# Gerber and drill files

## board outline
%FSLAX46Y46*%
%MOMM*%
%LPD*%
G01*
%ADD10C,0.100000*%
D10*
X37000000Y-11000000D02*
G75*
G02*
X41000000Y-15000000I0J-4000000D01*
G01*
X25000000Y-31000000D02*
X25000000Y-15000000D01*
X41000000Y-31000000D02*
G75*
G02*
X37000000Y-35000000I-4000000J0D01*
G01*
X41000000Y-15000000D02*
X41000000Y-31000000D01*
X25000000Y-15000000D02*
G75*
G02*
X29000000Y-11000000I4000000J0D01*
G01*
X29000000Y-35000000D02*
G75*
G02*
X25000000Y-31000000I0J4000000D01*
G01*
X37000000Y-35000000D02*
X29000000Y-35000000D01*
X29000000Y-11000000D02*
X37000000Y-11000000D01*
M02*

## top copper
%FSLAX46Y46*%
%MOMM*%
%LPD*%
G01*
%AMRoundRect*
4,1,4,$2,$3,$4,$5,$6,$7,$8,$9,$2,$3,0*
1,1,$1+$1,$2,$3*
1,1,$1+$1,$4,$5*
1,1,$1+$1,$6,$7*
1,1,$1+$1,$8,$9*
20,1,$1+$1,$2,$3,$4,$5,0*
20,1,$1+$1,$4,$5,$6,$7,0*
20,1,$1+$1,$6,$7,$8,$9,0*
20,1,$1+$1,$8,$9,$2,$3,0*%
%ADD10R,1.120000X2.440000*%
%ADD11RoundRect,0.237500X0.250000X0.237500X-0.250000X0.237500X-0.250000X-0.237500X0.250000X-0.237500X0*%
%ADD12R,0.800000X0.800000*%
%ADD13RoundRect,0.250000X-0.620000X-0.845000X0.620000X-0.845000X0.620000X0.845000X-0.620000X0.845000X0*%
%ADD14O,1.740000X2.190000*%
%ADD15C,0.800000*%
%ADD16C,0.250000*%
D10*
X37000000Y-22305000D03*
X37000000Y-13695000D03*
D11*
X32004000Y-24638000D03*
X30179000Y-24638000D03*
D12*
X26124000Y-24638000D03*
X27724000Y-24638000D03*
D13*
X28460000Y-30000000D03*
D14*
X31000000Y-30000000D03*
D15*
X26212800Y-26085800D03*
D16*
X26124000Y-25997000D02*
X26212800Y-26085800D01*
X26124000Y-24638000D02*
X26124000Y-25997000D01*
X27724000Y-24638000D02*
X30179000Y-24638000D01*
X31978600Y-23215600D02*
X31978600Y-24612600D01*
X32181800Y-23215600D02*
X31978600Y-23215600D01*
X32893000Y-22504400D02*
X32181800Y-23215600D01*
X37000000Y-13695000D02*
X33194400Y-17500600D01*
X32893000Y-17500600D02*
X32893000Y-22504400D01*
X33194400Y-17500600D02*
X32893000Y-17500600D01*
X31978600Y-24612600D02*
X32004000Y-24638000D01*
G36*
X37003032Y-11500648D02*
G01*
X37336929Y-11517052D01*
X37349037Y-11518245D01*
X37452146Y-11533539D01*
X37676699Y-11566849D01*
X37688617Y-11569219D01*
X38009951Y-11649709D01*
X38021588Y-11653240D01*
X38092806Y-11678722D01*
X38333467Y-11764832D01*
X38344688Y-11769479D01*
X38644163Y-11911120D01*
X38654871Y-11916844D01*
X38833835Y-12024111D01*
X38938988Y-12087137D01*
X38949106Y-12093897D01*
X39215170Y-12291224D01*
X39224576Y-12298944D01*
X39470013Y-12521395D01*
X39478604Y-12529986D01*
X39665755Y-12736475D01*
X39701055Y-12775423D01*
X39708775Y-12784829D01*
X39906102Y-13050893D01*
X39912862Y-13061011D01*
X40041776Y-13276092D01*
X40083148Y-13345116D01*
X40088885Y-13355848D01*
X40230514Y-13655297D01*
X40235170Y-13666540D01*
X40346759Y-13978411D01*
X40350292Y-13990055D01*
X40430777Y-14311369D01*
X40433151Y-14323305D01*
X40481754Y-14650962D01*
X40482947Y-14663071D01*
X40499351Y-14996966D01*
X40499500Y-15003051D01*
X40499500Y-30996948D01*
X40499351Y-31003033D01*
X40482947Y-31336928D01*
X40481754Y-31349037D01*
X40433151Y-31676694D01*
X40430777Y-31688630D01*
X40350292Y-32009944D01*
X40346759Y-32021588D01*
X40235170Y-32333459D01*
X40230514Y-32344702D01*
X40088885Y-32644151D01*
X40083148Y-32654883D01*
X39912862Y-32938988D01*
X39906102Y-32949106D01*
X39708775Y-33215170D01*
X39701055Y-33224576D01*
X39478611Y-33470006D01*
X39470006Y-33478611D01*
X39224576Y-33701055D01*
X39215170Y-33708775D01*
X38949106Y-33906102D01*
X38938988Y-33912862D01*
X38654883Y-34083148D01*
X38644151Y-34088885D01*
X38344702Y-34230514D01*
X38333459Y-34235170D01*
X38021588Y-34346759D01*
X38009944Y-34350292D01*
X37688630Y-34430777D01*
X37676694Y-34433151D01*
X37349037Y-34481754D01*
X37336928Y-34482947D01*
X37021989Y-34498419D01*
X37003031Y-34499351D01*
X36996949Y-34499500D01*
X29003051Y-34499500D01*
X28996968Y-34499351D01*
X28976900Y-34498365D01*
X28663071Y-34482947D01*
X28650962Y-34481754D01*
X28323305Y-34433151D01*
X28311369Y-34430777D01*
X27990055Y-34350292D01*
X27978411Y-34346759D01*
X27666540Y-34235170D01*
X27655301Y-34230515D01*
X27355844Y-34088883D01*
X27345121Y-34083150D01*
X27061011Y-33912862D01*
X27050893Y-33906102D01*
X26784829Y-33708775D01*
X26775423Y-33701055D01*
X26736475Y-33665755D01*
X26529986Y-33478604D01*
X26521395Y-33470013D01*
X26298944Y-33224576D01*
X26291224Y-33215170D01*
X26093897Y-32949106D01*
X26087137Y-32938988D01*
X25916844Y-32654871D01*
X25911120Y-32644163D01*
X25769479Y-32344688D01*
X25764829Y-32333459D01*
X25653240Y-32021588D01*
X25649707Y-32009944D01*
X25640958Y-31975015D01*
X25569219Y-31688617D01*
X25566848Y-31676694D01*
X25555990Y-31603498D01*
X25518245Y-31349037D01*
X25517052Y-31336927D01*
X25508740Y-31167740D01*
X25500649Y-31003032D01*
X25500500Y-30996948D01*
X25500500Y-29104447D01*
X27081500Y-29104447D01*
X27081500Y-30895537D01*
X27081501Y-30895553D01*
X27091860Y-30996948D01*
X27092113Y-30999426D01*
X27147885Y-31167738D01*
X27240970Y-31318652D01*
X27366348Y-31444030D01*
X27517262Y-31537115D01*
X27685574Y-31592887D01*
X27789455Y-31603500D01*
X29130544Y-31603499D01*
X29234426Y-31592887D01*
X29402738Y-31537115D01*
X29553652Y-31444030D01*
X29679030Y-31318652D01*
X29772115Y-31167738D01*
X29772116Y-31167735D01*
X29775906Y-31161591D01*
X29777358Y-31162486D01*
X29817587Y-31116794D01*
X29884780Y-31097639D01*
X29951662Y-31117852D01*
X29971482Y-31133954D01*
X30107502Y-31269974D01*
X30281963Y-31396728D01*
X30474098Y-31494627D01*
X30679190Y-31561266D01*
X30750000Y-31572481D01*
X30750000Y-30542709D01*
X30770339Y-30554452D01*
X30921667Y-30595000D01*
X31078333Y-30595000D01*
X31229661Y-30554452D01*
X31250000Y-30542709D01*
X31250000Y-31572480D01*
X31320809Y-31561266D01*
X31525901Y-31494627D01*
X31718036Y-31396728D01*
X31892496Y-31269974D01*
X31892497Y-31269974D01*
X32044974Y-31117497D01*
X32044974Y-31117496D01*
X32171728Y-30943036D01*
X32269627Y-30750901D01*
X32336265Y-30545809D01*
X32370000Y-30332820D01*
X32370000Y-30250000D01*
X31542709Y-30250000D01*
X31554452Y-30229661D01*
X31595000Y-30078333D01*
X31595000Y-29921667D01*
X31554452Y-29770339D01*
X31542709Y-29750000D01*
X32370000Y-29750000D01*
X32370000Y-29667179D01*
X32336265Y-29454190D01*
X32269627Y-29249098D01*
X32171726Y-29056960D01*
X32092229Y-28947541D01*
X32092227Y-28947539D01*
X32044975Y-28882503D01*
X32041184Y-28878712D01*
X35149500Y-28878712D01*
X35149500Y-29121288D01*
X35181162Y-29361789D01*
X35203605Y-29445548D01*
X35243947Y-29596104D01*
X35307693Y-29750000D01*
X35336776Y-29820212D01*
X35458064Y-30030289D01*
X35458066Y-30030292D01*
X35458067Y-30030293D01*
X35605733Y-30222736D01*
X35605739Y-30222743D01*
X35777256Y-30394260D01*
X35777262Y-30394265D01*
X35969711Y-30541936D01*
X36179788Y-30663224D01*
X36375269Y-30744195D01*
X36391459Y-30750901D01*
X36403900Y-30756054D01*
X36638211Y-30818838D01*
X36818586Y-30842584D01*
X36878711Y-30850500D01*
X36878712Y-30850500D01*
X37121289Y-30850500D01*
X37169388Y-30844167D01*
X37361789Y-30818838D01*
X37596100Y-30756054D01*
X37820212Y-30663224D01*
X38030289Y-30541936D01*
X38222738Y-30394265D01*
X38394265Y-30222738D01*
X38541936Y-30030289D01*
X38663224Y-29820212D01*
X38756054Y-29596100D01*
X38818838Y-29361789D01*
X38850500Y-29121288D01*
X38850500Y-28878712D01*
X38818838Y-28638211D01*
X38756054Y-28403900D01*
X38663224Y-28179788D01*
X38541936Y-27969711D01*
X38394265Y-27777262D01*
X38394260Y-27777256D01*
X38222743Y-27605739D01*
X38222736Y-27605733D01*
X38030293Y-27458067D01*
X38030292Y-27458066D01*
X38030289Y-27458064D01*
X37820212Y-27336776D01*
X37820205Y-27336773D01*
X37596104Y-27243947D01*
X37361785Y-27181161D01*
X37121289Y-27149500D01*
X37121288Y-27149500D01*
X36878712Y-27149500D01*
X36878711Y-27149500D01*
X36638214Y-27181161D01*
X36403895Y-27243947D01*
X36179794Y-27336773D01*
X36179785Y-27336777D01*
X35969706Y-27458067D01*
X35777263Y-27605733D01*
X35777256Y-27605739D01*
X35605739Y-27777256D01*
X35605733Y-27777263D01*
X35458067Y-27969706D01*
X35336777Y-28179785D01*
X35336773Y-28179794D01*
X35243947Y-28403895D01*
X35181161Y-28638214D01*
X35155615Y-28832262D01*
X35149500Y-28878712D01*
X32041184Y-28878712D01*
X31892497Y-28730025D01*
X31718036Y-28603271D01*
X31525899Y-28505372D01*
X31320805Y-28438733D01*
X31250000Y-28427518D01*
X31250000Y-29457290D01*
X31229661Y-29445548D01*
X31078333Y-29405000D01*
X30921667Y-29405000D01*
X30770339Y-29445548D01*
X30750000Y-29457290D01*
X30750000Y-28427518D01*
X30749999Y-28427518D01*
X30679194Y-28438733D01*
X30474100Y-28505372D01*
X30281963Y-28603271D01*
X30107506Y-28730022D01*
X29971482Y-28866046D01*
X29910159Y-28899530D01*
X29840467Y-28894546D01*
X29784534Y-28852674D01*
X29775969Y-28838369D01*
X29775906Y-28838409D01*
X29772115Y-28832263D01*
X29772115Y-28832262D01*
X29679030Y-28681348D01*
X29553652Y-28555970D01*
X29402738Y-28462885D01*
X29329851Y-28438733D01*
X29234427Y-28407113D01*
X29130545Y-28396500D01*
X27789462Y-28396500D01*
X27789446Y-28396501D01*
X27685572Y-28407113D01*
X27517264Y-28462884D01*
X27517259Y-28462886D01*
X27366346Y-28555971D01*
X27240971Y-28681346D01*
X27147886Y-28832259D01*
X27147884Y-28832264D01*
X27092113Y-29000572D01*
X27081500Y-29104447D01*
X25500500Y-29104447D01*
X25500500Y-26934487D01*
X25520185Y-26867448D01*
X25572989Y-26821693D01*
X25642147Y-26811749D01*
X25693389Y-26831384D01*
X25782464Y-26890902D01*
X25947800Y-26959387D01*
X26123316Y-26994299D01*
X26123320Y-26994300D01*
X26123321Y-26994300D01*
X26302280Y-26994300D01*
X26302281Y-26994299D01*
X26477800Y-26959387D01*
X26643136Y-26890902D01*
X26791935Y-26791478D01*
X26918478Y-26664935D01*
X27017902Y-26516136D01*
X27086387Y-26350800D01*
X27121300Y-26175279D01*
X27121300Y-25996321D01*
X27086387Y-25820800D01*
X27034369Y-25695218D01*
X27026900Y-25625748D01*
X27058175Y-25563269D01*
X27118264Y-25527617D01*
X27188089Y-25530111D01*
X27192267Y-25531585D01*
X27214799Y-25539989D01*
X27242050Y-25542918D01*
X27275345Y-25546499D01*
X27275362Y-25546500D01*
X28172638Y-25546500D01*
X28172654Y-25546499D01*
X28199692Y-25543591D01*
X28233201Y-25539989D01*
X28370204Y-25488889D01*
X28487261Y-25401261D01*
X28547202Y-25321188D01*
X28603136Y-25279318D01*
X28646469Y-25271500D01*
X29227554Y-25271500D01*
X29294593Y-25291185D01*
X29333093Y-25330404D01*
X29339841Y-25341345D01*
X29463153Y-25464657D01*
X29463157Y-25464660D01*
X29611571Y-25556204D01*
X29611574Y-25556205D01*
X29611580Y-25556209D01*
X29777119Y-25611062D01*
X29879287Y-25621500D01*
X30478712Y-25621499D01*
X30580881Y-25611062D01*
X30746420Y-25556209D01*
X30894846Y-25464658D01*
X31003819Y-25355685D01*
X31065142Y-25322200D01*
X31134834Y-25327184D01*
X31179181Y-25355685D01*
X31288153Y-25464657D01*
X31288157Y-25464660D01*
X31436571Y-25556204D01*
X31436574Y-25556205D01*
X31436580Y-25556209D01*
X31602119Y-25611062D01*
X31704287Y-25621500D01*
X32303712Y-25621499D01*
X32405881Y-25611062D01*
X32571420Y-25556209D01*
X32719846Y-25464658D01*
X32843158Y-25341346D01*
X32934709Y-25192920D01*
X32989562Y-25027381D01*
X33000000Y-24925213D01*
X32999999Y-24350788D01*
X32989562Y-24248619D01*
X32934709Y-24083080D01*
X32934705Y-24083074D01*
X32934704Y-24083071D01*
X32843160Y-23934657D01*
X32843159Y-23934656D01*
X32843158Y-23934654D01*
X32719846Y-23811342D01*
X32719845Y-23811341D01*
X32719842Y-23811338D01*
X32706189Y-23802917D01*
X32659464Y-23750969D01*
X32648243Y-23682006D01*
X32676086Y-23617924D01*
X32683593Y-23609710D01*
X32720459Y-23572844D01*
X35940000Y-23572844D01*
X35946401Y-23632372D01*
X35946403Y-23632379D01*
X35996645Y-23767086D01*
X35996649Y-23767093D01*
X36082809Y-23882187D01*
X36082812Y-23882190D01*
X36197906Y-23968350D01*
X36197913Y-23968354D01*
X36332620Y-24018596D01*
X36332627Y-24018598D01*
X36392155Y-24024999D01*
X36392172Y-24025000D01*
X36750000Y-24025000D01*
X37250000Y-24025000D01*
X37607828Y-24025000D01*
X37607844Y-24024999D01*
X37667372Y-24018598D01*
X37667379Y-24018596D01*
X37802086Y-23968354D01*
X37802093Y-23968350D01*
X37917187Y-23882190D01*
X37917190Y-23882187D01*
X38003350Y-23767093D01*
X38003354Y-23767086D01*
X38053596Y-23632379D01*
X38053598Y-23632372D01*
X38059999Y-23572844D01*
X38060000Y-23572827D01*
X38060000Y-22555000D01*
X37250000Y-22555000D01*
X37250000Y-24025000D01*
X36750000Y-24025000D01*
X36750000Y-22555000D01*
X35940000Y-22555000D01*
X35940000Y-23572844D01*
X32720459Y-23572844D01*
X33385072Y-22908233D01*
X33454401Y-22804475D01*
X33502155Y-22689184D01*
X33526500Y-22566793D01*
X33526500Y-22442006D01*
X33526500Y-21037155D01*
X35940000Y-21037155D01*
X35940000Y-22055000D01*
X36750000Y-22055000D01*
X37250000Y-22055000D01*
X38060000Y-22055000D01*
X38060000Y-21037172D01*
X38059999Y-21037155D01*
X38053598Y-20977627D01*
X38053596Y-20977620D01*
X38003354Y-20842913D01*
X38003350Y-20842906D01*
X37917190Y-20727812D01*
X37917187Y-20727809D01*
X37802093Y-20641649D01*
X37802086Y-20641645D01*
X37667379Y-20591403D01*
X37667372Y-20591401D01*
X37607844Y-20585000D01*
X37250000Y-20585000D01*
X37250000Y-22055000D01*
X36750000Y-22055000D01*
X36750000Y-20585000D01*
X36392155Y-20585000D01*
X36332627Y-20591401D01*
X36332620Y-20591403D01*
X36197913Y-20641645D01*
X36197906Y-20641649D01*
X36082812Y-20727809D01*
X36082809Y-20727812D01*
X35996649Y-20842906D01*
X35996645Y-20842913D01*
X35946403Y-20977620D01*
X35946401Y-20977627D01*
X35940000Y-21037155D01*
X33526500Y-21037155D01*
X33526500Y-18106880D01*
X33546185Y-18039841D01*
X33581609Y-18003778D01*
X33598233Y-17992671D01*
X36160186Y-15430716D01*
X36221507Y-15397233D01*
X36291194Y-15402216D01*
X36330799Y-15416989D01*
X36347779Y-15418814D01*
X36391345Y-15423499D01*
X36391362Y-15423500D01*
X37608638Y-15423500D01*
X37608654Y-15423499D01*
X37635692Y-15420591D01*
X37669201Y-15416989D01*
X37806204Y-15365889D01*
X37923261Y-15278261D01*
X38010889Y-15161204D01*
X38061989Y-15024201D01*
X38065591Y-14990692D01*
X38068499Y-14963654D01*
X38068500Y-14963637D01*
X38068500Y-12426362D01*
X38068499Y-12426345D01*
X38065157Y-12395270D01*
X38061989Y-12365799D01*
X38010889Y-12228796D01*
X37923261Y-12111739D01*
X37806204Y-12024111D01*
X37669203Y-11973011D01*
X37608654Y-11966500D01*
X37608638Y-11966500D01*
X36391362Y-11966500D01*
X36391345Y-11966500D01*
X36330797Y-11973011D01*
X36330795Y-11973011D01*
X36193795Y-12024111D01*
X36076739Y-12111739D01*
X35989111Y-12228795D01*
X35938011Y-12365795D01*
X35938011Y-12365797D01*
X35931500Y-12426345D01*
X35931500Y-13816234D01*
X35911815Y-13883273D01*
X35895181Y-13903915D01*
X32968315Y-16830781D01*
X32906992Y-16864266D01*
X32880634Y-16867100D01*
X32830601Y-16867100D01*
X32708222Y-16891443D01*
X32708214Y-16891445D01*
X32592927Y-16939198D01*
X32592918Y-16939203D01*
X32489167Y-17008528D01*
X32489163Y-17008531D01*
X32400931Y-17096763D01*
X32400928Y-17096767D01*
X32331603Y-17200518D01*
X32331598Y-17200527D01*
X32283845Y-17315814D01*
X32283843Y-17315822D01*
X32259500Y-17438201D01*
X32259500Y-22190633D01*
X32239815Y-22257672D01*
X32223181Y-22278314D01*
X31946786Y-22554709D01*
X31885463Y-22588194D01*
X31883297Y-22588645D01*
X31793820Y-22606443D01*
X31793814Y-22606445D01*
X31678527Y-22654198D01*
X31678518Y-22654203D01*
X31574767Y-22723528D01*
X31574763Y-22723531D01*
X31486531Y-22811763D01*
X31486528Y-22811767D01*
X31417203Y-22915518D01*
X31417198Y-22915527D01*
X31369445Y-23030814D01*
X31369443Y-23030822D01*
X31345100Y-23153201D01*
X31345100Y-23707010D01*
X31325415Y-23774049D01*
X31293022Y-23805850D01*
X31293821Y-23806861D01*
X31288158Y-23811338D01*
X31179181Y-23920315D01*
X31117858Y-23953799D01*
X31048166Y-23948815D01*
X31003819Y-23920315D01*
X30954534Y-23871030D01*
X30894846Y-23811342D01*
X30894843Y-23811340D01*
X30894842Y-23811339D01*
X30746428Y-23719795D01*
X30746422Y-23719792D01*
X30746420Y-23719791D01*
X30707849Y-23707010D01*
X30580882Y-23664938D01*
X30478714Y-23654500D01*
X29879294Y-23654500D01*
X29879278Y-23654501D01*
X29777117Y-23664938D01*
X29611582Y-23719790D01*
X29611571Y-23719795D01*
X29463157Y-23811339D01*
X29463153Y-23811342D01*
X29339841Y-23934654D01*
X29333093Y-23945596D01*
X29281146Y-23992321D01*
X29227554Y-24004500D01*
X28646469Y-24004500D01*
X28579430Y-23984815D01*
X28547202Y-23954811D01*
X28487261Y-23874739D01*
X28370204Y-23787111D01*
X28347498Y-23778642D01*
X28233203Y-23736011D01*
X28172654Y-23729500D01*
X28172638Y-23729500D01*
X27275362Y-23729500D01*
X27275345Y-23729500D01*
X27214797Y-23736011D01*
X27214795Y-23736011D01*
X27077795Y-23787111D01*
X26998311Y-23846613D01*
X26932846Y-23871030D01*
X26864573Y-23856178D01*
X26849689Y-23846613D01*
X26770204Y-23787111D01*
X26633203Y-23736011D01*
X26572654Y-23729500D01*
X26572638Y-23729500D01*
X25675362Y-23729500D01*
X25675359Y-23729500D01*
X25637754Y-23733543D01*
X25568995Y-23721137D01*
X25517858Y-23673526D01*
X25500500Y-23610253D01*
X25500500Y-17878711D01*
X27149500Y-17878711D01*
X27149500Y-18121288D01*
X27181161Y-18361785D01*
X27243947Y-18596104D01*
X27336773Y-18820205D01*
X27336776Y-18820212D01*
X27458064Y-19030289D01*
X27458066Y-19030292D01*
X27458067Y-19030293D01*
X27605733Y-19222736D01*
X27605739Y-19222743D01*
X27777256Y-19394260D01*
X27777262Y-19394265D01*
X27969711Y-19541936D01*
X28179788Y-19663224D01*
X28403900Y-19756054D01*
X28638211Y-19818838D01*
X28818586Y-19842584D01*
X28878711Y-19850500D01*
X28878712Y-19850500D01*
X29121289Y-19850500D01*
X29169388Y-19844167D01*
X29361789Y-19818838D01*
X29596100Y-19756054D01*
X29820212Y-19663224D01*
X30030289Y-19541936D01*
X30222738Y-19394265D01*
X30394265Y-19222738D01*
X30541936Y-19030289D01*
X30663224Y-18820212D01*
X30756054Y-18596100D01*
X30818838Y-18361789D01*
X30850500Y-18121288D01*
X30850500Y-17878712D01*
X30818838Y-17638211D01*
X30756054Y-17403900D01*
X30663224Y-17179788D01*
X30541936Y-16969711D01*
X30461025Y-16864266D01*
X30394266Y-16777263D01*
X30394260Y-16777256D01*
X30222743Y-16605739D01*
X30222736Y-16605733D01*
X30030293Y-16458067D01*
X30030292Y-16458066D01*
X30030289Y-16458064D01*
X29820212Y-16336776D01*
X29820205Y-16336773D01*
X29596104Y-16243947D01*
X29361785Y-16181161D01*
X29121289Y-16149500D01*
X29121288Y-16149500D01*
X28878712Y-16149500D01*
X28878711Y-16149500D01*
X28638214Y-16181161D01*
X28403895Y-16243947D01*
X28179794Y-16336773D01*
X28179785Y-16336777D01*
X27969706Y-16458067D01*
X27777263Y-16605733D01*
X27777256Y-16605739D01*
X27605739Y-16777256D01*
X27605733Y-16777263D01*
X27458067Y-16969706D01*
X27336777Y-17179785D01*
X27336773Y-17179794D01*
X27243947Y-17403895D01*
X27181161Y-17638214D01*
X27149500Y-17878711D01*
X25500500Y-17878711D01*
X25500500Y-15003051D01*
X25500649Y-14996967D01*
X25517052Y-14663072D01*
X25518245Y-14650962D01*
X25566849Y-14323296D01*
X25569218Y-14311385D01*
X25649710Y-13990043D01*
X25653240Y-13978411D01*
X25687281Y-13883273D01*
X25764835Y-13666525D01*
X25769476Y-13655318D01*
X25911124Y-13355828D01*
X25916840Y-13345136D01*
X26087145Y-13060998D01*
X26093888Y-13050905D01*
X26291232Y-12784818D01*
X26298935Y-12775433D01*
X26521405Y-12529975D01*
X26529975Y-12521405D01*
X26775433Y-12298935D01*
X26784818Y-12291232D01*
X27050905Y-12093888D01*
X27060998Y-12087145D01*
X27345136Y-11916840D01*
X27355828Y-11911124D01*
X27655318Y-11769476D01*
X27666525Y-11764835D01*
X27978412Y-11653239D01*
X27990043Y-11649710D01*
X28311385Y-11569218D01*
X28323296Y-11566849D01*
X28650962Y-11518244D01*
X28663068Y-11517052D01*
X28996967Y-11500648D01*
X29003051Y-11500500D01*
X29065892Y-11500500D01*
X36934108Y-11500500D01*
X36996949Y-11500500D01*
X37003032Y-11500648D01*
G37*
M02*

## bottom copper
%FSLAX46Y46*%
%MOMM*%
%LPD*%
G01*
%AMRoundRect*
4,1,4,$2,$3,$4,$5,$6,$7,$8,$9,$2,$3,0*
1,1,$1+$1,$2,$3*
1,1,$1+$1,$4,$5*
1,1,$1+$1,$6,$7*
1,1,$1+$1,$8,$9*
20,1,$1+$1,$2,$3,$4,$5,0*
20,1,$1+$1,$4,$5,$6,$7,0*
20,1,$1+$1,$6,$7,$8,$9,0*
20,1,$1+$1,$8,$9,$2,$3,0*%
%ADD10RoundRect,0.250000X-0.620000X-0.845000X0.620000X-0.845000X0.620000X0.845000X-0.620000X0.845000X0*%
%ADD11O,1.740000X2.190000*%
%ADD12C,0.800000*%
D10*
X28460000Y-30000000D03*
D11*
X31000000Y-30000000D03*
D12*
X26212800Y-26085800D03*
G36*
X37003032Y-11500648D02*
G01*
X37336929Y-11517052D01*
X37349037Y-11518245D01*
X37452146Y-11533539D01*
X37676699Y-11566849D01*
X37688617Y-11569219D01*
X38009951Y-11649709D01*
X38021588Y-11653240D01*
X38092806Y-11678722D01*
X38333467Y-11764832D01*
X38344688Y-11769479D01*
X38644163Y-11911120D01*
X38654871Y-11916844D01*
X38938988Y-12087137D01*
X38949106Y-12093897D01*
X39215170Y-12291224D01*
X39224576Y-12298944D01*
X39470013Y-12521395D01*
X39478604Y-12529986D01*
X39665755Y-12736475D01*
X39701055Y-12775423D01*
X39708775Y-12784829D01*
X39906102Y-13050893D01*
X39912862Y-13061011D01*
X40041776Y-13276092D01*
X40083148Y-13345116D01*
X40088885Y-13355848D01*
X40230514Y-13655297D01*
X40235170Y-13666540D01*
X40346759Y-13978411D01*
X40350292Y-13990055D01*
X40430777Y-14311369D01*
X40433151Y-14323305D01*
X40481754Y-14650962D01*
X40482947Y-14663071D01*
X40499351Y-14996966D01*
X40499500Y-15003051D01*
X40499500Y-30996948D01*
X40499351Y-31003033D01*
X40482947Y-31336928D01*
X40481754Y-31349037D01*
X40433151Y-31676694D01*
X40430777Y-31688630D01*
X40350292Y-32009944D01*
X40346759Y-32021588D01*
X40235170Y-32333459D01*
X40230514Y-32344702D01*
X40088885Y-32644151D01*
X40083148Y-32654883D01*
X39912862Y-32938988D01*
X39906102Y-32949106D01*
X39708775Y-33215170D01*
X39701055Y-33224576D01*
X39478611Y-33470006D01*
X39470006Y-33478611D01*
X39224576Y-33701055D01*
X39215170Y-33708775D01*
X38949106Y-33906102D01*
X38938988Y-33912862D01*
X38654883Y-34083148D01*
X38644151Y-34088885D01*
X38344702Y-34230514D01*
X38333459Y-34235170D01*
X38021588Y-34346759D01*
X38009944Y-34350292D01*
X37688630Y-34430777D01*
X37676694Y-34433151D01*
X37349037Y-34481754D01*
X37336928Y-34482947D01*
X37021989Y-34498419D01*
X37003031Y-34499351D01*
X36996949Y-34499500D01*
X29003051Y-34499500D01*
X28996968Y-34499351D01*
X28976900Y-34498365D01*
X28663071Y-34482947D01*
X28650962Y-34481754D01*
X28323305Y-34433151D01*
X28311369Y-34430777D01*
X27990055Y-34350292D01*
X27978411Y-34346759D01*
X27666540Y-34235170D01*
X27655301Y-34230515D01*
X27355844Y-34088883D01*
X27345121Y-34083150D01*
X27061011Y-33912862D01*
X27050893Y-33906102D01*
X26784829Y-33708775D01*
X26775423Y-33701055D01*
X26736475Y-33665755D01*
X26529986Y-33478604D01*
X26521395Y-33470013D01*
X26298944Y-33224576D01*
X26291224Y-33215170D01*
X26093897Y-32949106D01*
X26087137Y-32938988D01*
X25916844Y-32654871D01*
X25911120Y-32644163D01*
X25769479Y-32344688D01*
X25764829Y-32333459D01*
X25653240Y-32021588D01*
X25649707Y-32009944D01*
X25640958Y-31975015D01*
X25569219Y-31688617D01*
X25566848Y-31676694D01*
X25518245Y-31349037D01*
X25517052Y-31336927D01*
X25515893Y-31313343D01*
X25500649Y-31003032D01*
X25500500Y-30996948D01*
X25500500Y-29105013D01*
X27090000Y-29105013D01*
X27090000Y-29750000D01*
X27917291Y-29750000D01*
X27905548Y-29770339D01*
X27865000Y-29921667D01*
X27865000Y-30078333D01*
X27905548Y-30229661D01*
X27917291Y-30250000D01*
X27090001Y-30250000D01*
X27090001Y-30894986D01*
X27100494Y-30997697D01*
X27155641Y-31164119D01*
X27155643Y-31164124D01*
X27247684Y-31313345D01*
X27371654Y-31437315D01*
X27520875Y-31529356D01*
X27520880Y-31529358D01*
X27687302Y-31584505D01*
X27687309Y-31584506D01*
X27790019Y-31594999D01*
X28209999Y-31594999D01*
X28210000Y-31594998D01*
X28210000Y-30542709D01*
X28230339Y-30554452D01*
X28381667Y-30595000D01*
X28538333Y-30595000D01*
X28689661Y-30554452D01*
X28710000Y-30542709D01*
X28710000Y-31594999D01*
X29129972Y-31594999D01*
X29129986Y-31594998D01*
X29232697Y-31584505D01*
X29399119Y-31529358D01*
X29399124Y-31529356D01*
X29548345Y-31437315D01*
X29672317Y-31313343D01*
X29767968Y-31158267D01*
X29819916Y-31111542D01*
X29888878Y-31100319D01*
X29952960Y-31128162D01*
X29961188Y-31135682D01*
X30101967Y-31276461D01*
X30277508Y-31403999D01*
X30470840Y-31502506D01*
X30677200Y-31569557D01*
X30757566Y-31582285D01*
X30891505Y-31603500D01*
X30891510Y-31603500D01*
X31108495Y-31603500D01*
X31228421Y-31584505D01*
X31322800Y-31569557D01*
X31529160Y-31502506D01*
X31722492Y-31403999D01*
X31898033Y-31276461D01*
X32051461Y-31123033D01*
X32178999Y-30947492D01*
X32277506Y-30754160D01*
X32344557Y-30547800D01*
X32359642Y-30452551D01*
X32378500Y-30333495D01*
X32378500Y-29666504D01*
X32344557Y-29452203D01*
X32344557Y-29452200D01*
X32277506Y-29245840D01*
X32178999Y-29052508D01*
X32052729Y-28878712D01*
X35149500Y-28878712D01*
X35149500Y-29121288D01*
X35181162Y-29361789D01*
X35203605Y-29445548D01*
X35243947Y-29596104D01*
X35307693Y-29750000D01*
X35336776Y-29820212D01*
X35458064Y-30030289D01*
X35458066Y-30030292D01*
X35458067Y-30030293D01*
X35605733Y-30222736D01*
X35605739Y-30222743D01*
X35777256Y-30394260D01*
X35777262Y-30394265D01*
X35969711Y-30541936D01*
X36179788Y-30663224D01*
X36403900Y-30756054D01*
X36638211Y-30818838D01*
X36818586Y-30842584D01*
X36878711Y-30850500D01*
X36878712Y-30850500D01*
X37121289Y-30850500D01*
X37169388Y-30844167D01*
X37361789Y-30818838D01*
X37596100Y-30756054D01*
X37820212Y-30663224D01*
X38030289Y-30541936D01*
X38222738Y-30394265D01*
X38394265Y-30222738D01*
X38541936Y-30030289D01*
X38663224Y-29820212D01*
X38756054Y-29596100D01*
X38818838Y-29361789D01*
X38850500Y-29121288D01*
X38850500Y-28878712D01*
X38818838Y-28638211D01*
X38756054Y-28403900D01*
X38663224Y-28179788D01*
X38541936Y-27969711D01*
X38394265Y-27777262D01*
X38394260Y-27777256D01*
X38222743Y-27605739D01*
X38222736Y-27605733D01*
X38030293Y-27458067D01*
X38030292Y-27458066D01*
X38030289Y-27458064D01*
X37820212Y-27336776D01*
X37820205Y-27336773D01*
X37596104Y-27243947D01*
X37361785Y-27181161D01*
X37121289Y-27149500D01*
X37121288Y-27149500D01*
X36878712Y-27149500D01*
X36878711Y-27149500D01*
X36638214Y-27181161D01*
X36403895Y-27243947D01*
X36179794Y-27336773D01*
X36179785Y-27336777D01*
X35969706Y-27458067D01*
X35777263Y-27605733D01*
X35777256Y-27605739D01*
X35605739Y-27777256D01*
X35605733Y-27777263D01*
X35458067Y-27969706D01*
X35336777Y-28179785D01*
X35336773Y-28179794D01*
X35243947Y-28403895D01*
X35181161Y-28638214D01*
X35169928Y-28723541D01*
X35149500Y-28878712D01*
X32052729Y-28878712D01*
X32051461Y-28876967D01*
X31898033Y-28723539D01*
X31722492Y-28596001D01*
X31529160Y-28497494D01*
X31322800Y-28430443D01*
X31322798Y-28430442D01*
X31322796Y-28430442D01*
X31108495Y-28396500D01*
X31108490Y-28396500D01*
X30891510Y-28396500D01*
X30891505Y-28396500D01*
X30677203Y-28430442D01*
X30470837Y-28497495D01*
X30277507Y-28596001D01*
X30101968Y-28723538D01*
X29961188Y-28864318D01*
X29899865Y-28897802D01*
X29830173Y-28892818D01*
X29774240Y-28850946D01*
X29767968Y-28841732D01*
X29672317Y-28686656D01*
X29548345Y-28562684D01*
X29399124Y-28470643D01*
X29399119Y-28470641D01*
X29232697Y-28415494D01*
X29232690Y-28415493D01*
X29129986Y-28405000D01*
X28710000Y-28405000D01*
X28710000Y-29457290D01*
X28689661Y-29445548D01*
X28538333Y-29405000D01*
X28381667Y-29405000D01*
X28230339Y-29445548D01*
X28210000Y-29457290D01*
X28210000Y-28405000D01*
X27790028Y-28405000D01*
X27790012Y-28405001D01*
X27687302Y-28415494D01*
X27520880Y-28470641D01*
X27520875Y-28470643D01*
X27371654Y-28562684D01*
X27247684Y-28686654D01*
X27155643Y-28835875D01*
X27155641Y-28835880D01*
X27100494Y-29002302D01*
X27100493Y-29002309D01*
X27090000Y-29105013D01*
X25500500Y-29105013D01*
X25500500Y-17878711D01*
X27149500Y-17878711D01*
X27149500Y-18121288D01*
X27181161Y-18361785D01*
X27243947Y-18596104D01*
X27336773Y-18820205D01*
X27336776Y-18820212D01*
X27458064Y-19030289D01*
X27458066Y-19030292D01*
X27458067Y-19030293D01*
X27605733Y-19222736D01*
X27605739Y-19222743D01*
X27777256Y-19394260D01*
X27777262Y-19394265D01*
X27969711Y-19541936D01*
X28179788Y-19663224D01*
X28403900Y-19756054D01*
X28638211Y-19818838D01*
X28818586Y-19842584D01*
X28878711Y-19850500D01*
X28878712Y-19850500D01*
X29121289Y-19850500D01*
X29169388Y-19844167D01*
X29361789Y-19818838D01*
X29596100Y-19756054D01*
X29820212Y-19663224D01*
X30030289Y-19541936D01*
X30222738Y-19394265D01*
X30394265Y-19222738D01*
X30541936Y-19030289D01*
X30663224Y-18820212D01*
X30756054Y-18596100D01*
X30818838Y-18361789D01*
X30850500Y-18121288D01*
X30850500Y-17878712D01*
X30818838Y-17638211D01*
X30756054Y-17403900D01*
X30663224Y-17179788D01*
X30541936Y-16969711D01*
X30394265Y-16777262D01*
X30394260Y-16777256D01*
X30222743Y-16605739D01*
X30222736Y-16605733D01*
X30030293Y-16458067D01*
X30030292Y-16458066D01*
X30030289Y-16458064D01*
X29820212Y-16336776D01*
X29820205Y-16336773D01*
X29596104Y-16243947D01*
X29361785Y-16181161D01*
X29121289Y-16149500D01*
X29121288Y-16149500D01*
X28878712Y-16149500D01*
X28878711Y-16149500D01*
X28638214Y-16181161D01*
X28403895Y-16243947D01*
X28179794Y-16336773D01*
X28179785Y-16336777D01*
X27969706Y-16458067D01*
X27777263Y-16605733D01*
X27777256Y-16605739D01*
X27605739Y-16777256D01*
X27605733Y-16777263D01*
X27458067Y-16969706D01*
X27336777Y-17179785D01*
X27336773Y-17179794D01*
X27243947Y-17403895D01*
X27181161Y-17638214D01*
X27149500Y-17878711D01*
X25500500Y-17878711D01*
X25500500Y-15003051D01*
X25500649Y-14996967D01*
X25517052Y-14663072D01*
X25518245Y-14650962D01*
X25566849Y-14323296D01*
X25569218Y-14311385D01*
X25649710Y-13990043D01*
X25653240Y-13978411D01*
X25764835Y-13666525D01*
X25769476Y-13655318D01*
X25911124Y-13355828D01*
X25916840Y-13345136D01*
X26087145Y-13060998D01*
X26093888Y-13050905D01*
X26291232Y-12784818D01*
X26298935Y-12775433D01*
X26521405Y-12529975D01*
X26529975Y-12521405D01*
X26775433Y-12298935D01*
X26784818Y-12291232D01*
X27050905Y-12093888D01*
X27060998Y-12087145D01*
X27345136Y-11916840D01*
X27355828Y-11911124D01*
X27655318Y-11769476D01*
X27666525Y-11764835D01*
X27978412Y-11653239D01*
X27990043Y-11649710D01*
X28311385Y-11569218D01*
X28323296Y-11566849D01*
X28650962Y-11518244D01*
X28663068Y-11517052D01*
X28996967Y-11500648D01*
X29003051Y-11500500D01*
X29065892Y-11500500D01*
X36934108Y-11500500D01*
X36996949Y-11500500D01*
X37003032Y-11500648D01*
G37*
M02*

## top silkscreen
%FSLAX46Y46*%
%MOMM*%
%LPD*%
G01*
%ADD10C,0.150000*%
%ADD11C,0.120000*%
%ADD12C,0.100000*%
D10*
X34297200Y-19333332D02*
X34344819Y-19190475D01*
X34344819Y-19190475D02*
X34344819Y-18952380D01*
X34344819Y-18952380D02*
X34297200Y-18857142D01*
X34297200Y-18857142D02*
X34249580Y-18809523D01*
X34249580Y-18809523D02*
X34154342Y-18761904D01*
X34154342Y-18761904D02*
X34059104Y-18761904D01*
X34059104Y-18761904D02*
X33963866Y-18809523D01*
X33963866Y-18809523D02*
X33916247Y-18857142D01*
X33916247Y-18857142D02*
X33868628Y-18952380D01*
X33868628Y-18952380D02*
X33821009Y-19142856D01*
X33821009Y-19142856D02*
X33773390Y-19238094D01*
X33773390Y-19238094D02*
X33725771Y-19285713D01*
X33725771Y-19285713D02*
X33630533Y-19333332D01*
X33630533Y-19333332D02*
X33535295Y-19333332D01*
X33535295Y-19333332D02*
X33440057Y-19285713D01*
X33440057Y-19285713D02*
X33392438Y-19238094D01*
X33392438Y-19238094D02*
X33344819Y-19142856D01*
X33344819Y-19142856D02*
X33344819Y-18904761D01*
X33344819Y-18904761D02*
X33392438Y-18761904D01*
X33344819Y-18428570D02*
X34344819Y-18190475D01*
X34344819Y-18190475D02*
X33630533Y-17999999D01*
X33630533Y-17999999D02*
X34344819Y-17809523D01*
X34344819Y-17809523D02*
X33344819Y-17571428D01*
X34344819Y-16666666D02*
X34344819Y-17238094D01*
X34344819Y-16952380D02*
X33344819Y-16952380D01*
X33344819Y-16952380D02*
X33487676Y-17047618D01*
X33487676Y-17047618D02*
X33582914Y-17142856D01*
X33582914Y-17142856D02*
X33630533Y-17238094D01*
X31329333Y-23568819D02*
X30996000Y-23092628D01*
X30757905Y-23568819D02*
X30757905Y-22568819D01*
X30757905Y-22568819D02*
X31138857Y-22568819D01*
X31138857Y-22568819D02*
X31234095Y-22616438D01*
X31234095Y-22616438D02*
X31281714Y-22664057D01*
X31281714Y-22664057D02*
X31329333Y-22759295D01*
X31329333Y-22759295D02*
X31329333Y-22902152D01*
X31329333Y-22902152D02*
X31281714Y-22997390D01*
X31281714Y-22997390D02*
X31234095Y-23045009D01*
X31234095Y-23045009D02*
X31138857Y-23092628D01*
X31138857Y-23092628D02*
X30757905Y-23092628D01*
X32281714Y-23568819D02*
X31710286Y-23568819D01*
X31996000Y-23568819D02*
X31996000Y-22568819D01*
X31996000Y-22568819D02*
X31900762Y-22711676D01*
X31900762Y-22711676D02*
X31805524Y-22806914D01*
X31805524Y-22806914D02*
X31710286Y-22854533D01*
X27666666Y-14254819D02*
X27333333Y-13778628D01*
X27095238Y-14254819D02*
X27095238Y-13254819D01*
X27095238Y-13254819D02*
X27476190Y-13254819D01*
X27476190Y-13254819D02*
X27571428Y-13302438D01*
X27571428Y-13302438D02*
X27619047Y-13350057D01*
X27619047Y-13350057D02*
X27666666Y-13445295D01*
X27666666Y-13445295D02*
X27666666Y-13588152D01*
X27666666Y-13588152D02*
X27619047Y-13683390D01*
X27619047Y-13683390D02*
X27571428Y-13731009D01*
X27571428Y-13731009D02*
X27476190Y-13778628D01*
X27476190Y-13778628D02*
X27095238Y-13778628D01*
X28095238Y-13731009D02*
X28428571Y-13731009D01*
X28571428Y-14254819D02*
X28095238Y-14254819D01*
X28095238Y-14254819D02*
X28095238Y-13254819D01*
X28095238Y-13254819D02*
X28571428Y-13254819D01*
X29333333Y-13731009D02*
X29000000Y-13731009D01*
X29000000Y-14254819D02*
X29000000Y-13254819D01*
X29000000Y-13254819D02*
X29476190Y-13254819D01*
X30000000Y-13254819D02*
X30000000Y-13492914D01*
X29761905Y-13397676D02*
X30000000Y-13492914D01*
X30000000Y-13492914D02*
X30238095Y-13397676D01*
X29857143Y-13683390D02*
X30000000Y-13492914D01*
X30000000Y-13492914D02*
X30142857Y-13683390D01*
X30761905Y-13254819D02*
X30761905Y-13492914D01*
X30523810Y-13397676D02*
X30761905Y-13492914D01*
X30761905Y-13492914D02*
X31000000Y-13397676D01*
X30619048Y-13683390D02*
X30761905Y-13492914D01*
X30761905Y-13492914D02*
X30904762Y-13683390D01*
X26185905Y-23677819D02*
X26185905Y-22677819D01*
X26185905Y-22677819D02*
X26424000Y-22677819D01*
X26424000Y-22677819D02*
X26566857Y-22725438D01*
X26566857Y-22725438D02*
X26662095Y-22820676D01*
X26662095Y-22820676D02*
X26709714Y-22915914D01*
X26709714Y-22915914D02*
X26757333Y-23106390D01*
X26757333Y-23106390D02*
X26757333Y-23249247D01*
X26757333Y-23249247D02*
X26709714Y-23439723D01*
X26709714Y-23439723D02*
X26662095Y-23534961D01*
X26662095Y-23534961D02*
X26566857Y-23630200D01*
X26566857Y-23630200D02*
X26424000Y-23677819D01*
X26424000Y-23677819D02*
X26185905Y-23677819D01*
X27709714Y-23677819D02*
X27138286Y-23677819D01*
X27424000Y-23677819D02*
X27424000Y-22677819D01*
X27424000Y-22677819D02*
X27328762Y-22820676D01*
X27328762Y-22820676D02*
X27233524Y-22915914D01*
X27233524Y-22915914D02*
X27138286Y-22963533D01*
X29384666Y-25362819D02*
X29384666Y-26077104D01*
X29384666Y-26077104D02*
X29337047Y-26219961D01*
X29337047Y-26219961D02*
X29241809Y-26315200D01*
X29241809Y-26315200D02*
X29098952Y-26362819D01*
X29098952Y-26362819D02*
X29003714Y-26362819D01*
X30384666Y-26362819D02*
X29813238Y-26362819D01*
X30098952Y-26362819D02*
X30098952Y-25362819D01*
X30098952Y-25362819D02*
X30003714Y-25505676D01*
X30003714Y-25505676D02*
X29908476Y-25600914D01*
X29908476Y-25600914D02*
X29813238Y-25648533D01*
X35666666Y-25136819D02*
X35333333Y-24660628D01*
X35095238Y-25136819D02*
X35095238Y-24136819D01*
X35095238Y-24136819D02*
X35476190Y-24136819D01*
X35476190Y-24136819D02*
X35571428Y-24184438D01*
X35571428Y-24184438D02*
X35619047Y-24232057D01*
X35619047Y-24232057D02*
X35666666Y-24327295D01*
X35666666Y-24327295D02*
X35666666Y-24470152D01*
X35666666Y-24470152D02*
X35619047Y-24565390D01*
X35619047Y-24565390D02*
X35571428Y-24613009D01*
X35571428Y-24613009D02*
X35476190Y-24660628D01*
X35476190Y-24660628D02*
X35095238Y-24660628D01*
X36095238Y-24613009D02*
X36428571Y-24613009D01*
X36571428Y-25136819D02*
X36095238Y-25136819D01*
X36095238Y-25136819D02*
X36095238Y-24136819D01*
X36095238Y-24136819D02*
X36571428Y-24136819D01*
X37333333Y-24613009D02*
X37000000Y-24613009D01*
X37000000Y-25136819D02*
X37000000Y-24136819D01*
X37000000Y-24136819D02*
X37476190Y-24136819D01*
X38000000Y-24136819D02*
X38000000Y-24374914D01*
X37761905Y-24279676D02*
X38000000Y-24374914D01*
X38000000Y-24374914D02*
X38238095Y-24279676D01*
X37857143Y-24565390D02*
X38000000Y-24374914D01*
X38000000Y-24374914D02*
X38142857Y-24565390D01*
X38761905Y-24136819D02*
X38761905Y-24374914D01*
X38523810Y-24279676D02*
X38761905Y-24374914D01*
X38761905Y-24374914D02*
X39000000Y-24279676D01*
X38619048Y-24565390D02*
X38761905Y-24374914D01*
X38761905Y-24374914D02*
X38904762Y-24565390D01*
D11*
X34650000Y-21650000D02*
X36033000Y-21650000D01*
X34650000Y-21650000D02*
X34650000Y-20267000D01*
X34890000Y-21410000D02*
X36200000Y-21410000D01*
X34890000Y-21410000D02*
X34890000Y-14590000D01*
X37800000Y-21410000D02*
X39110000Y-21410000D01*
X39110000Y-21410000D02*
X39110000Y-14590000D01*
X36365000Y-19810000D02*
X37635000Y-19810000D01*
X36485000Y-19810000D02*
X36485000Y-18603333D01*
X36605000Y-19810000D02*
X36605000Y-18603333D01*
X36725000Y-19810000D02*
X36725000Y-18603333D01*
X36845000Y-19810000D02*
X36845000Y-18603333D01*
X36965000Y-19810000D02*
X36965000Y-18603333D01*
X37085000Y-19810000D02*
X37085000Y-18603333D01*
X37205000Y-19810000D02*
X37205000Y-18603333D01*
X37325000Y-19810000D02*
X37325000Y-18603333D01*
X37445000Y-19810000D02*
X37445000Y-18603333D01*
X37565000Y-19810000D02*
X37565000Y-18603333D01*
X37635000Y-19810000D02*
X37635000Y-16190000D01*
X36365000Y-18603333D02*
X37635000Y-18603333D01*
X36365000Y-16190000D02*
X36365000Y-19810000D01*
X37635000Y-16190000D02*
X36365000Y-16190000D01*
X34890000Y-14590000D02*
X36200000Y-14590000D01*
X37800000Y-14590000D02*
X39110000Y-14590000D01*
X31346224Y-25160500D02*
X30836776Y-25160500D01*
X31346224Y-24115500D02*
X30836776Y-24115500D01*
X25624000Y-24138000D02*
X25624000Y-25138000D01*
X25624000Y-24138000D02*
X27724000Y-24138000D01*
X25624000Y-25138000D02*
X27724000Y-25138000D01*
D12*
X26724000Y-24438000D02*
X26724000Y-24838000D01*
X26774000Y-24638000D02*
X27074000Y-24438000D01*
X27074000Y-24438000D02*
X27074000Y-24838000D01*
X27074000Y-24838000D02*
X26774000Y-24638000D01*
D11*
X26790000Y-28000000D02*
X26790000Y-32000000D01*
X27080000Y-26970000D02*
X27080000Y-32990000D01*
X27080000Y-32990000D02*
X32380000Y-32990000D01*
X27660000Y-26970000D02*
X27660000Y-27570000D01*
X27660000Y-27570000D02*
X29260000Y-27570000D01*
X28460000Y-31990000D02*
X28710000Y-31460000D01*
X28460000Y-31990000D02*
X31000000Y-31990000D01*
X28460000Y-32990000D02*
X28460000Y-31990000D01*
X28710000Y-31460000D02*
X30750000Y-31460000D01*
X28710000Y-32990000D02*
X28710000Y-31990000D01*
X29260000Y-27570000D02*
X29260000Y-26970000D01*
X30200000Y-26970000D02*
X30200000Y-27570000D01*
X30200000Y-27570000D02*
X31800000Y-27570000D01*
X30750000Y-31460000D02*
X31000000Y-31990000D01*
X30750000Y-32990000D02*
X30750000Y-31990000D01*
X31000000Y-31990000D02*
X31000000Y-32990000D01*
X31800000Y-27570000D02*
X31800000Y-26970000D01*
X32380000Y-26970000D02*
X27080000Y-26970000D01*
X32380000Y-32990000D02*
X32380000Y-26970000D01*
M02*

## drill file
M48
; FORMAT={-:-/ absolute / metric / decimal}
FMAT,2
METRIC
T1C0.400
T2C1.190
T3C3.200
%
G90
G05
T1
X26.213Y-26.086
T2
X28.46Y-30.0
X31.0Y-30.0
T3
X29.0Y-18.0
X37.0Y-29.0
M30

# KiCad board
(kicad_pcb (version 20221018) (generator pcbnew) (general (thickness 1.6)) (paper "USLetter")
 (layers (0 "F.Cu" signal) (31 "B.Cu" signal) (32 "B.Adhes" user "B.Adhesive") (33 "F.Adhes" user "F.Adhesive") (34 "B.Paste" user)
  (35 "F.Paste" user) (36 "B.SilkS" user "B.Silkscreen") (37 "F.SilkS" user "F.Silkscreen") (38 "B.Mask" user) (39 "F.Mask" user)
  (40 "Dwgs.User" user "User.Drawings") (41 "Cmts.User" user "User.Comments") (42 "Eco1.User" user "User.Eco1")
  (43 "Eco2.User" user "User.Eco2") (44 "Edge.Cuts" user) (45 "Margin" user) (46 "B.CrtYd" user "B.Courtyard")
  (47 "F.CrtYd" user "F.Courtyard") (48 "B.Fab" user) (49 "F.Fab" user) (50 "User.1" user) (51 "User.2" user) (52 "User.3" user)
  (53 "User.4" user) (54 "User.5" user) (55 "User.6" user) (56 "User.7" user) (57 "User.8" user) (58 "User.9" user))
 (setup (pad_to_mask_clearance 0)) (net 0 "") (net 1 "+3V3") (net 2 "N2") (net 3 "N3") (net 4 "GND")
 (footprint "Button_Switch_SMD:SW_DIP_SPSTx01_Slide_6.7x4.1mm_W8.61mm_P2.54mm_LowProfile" (layer "F.Cu") (at 37 18 90)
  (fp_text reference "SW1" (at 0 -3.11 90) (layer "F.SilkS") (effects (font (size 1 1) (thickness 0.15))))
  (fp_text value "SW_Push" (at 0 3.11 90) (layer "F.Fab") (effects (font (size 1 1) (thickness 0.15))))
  (fp_line (start -3.65 -2.35) (end -3.65 -0.967) (stroke (width 0.12) (type solid)) (layer "F.SilkS"))
  (fp_line (start -3.65 -2.35) (end -2.267 -2.35) (stroke (width 0.12) (type solid)) (layer "F.SilkS"))
  (fp_line (start -3.41 -2.11) (end -3.41 -0.8) (stroke (width 0.12) (type solid)) (layer "F.SilkS"))
  (fp_line (start -3.41 -2.11) (end 3.41 -2.11) (stroke (width 0.12) (type solid)) (layer "F.SilkS"))
  (fp_line (start -3.41 0.8) (end -3.41 2.11) (stroke (width 0.12) (type solid)) (layer "F.SilkS"))
  (fp_line (start -3.41 2.11) (end 3.41 2.11) (stroke (width 0.12) (type solid)) (layer "F.SilkS"))
  (fp_line (start -1.81 -0.635) (end -1.81 0.635) (stroke (width 0.12) (type solid)) (layer "F.SilkS"))
  (fp_line (start -1.81 -0.515) (end -0.603333 -0.515) (stroke (width 0.12) (type solid)) (layer "F.SilkS"))
  (fp_line (start -1.81 -0.395) (end -0.603333 -0.395) (stroke (width 0.12) (type solid)) (layer "F.SilkS"))
  (fp_line (start -1.81 -0.275) (end -0.603333 -0.275) (stroke (width 0.12) (type solid)) (layer "F.SilkS"))
  (fp_line (start -1.81 -0.155) (end -0.603333 -0.155) (stroke (width 0.12) (type solid)) (layer "F.SilkS"))
  (fp_line (start -1.81 -0.035) (end -0.603333 -0.035) (stroke (width 0.12) (type solid)) (layer "F.SilkS"))
  (fp_line (start -1.81 0.085) (end -0.603333 0.085) (stroke (width 0.12) (type solid)) (layer "F.SilkS"))
  (fp_line (start -1.81 0.205) (end -0.603333 0.205) (stroke (width 0.12) (type solid)) (layer "F.SilkS"))
  (fp_line (start -1.81 0.325) (end -0.603333 0.325) (stroke (width 0.12) (type solid)) (layer "F.SilkS"))
  (fp_line (start -1.81 0.445) (end -0.603333 0.445) (stroke (width 0.12) (type solid)) (layer "F.SilkS"))
  (fp_line (start -1.81 0.565) (end -0.603333 0.565) (stroke (width 0.12) (type solid)) (layer "F.SilkS"))
  (fp_line (start -1.81 0.635) (end 1.81 0.635) (stroke (width 0.12) (type solid)) (layer "F.SilkS"))
  (fp_line (start -0.603333 -0.635) (end -0.603333 0.635) (stroke (width 0.12) (type solid)) (layer "F.SilkS"))
  (fp_line (start 1.81 -0.635) (end -1.81 -0.635) (stroke (width 0.12) (type solid)) (layer "F.SilkS"))
  (fp_line (start 1.81 0.635) (end 1.81 -0.635) (stroke (width 0.12) (type solid)) (layer "F.SilkS"))
  (fp_line (start 3.41 -2.11) (end 3.41 -0.8) (stroke (width 0.12) (type solid)) (layer "F.SilkS"))
  (fp_line (start 3.41 0.8) (end 3.41 2.11) (stroke (width 0.12) (type solid)) (layer "F.SilkS"))
  (pad "1" smd rect (at -4.305 0 90) (size 2.44 1.12) (layers "F.Cu" "F.Paste" "F.Mask") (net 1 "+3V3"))
  (pad "2" smd rect (at 4.305 0 90) (size 2.44 1.12) (layers "F.Cu" "F.Paste" "F.Mask") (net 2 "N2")))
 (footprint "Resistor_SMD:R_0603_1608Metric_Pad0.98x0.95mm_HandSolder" (layer "F.Cu") (at 31.0915 24.638 180)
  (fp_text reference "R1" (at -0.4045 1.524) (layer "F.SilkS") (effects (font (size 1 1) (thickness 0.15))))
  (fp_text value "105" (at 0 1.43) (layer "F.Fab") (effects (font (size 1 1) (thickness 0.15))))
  (fp_line (start -0.254724 -0.5225) (end 0.254724 -0.5225) (stroke (width 0.12) (type solid)) (layer "F.SilkS"))
  (fp_line (start -0.254724 0.5225) (end 0.254724 0.5225) (stroke (width 0.12) (type solid)) (layer "F.SilkS"))
  (pad "1" smd roundrect (at -0.9125 0 180) (size 0.975 0.95) (layers "F.Cu" "F.Paste" "F.Mask") (roundrect_rratio 0.25) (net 2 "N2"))
  (pad "2" smd roundrect (at 0.9125 0 180) (size 0.975 0.95) (layers "F.Cu" "F.Paste" "F.Mask") (roundrect_rratio 0.25) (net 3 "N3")))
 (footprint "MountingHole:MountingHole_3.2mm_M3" (layer "F.Cu") (at 29 18)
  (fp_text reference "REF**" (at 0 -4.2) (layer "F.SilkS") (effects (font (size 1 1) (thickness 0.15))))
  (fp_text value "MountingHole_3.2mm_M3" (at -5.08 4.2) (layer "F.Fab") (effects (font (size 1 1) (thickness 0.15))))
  (pad "" np_thru_hole circle (at 0 0) (size 3.2 3.2) (drill 3.2) (layers "*.Cu" "*.Mask")))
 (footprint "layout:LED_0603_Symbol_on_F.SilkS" (layer "F.Cu") (at 26.924 24.638)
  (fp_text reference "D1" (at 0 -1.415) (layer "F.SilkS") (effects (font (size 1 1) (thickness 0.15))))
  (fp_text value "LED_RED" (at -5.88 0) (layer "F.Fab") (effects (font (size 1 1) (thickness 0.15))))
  (fp_line (start -1.3 -0.5) (end -1.3 0.5) (stroke (width 0.12) (type solid)) (layer "F.SilkS"))
  (fp_line (start -1.3 -0.5) (end 0.8 -0.5) (stroke (width 0.12) (type solid)) (layer "F.SilkS"))
  (fp_line (start -1.3 0.5) (end 0.8 0.5) (stroke (width 0.12) (type solid)) (layer "F.SilkS"))
  (fp_line (start -0.2 -0.2) (end -0.2 0.2) (stroke (width 0.1) (type solid)) (layer "F.SilkS"))
  (fp_line (start -0.15 0) (end 0.15 -0.2) (stroke (width 0.1) (type solid)) (layer "F.SilkS"))
  (fp_line (start 0.15 -0.2) (end 0.15 0.2) (stroke (width 0.1) (type solid)) (layer "F.SilkS"))
  (fp_line (start 0.15 0.2) (end -0.15 0) (stroke (width 0.1) (type solid)) (layer "F.SilkS"))
  (pad "1" smd rect (at -0.8 0 180) (size 0.8 0.8) (layers "F.Cu" "F.Paste" "F.Mask") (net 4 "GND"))
  (pad "2" smd rect (at 0.8 0 180) (size 0.8 0.8) (layers "F.Cu" "F.Paste" "F.Mask") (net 3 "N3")))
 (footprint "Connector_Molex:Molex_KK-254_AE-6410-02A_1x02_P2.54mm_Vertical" (layer "F.Cu") (at 28.46 30)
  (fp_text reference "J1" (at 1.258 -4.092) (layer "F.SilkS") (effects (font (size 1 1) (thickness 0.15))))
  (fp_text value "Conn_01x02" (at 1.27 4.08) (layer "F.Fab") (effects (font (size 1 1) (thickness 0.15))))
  (fp_line (start -1.67 -2) (end -1.67 2) (stroke (width 0.12) (type solid)) (layer "F.SilkS"))
  (fp_line (start -1.38 -3.03) (end -1.38 2.99) (stroke (width 0.12) (type solid)) (layer "F.SilkS"))
  (fp_line (start -1.38 2.99) (end 3.92 2.99) (stroke (width 0.12) (type solid)) (layer "F.SilkS"))
  (fp_line (start -0.8 -3.03) (end -0.8 -2.43) (stroke (width 0.12) (type solid)) (layer "F.SilkS"))
  (fp_line (start -0.8 -2.43) (end 0.8 -2.43) (stroke (width 0.12) (type solid)) (layer "F.SilkS"))
  (fp_line (start 0 1.99) (end 0.25 1.46) (stroke (width 0.12) (type solid)) (layer "F.SilkS"))
  (fp_line (start 0 1.99) (end 2.54 1.99) (stroke (width 0.12) (type solid)) (layer "F.SilkS"))
  (fp_line (start 0 2.99) (end 0 1.99) (stroke (width 0.12) (type solid)) (layer "F.SilkS"))
  (fp_line (start 0.25 1.46) (end 2.29 1.46) (stroke (width 0.12) (type solid)) (layer "F.SilkS"))
  (fp_line (start 0.25 2.99) (end 0.25 1.99) (stroke (width 0.12) (type solid)) (layer "F.SilkS"))
  (fp_line (start 0.8 -2.43) (end 0.8 -3.03) (stroke (width 0.12) (type solid)) (layer "F.SilkS"))
  (fp_line (start 1.74 -3.03) (end 1.74 -2.43) (stroke (width 0.12) (type solid)) (layer "F.SilkS"))
  (fp_line (start 1.74 -2.43) (end 3.34 -2.43) (stroke (width 0.12) (type solid)) (layer "F.SilkS"))
  (fp_line (start 2.29 1.46) (end 2.54 1.99) (stroke (width 0.12) (type solid)) (layer "F.SilkS"))
  (fp_line (start 2.29 2.99) (end 2.29 1.99) (stroke (width 0.12) (type solid)) (layer "F.SilkS"))
  (fp_line (start 2.54 1.99) (end 2.54 2.99) (stroke (width 0.12) (type solid)) (layer "F.SilkS"))
  (fp_line (start 3.34 -2.43) (end 3.34 -3.03) (stroke (width 0.12) (type solid)) (layer "F.SilkS"))
  (fp_line (start 3.92 -3.03) (end -1.38 -3.03) (stroke (width 0.12) (type solid)) (layer "F.SilkS"))
  (fp_line (start 3.92 2.99) (end 3.92 -3.03) (stroke (width 0.12) (type solid)) (layer "F.SilkS"))
  (pad "1" thru_hole roundrect (at 0 0) (size 1.74 2.19) (drill 1.19) (layers "*.Cu" "*.Mask") (roundrect_rratio 0.143678) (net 4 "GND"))
  (pad "2" thru_hole oval (at 2.54 0) (size 1.74 2.19) (drill 1.19) (layers "*.Cu" "*.Mask") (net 1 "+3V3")))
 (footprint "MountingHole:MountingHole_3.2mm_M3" (layer "F.Cu") (at 37 29)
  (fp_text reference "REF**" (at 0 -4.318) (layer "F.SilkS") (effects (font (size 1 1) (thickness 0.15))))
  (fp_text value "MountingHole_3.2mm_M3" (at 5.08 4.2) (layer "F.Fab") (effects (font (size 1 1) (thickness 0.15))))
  (pad "" np_thru_hole circle (at 0 0) (size 3.2 3.2) (drill 3.2) (layers "*.Cu" "*.Mask")))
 (gr_arc (start 37 11) (mid 39.828427 12.171573) (end 41 15) (stroke (width 0.1) (type default)) (layer "Edge.Cuts"))
 (gr_line (start 25 31) (end 25 15) (stroke (width 0.1) (type default)) (layer "Edge.Cuts"))
 (gr_arc (start 41 31) (mid 39.828427 33.828427) (end 37 35) (stroke (width 0.1) (type default)) (layer "Edge.Cuts"))
 (gr_line (start 41 15) (end 41 31) (stroke (width 0.1) (type default)) (layer "Edge.Cuts"))
 (gr_arc (start 25 15) (mid 26.171573 12.171573) (end 29 11) (stroke (width 0.1) (type default)) (layer "Edge.Cuts"))
 (gr_arc (start 29 35) (mid 26.171573 33.828427) (end 25 31) (stroke (width 0.1) (type default)) (layer "Edge.Cuts"))
 (gr_line (start 37 35) (end 29 35) (stroke (width 0.1) (type default)) (layer "Edge.Cuts"))
 (gr_line (start 29 11) (end 37 11) (stroke (width 0.1) (type default)) (layer "Edge.Cuts"))
 (segment (start 26.124 25.997) (end 26.2128 26.0858) (width 0.25) (layer "F.Cu") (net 4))
 (segment (start 26.124 24.638) (end 26.124 25.997) (width 0.25) (layer "F.Cu") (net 4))
 (via (at 26.2128 26.0858) (size 0.8) (drill 0.4) (layers "F.Cu" "B.Cu") (free) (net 4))
 (segment (start 27.724 24.638) (end 30.179 24.638) (width 0.25) (layer "F.Cu") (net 3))
 (segment (start 31.9786 23.2156) (end 31.9786 24.6126) (width 0.25) (layer "F.Cu") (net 2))
 (segment (start 32.1818 23.2156) (end 31.9786 23.2156) (width 0.25) (layer "F.Cu") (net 2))
 (segment (start 32.893 22.5044) (end 32.1818 23.2156) (width 0.25) (layer "F.Cu") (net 2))
 (segment (start 37 13.695) (end 33.1944 17.5006) (width 0.25) (layer "F.Cu") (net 2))
 (segment (start 32.893 17.5006) (end 32.893 22.5044) (width 0.25) (layer "F.Cu") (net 2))
 (segment (start 33.1944 17.5006) (end 32.893 17.5006) (width 0.25) (layer "F.Cu") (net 2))
 (segment (start 31.9786 24.6126) (end 32.004 24.638) (width 0.25) (layer "F.Cu") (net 2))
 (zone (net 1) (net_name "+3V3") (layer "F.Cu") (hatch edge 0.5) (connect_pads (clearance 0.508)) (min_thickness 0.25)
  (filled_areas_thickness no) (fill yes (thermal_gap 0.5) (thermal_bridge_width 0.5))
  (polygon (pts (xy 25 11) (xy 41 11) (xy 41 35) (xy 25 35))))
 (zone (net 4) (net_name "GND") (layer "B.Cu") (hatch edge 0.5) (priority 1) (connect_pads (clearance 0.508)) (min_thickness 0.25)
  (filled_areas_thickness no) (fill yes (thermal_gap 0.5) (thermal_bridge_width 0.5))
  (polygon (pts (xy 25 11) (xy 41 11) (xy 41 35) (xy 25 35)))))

